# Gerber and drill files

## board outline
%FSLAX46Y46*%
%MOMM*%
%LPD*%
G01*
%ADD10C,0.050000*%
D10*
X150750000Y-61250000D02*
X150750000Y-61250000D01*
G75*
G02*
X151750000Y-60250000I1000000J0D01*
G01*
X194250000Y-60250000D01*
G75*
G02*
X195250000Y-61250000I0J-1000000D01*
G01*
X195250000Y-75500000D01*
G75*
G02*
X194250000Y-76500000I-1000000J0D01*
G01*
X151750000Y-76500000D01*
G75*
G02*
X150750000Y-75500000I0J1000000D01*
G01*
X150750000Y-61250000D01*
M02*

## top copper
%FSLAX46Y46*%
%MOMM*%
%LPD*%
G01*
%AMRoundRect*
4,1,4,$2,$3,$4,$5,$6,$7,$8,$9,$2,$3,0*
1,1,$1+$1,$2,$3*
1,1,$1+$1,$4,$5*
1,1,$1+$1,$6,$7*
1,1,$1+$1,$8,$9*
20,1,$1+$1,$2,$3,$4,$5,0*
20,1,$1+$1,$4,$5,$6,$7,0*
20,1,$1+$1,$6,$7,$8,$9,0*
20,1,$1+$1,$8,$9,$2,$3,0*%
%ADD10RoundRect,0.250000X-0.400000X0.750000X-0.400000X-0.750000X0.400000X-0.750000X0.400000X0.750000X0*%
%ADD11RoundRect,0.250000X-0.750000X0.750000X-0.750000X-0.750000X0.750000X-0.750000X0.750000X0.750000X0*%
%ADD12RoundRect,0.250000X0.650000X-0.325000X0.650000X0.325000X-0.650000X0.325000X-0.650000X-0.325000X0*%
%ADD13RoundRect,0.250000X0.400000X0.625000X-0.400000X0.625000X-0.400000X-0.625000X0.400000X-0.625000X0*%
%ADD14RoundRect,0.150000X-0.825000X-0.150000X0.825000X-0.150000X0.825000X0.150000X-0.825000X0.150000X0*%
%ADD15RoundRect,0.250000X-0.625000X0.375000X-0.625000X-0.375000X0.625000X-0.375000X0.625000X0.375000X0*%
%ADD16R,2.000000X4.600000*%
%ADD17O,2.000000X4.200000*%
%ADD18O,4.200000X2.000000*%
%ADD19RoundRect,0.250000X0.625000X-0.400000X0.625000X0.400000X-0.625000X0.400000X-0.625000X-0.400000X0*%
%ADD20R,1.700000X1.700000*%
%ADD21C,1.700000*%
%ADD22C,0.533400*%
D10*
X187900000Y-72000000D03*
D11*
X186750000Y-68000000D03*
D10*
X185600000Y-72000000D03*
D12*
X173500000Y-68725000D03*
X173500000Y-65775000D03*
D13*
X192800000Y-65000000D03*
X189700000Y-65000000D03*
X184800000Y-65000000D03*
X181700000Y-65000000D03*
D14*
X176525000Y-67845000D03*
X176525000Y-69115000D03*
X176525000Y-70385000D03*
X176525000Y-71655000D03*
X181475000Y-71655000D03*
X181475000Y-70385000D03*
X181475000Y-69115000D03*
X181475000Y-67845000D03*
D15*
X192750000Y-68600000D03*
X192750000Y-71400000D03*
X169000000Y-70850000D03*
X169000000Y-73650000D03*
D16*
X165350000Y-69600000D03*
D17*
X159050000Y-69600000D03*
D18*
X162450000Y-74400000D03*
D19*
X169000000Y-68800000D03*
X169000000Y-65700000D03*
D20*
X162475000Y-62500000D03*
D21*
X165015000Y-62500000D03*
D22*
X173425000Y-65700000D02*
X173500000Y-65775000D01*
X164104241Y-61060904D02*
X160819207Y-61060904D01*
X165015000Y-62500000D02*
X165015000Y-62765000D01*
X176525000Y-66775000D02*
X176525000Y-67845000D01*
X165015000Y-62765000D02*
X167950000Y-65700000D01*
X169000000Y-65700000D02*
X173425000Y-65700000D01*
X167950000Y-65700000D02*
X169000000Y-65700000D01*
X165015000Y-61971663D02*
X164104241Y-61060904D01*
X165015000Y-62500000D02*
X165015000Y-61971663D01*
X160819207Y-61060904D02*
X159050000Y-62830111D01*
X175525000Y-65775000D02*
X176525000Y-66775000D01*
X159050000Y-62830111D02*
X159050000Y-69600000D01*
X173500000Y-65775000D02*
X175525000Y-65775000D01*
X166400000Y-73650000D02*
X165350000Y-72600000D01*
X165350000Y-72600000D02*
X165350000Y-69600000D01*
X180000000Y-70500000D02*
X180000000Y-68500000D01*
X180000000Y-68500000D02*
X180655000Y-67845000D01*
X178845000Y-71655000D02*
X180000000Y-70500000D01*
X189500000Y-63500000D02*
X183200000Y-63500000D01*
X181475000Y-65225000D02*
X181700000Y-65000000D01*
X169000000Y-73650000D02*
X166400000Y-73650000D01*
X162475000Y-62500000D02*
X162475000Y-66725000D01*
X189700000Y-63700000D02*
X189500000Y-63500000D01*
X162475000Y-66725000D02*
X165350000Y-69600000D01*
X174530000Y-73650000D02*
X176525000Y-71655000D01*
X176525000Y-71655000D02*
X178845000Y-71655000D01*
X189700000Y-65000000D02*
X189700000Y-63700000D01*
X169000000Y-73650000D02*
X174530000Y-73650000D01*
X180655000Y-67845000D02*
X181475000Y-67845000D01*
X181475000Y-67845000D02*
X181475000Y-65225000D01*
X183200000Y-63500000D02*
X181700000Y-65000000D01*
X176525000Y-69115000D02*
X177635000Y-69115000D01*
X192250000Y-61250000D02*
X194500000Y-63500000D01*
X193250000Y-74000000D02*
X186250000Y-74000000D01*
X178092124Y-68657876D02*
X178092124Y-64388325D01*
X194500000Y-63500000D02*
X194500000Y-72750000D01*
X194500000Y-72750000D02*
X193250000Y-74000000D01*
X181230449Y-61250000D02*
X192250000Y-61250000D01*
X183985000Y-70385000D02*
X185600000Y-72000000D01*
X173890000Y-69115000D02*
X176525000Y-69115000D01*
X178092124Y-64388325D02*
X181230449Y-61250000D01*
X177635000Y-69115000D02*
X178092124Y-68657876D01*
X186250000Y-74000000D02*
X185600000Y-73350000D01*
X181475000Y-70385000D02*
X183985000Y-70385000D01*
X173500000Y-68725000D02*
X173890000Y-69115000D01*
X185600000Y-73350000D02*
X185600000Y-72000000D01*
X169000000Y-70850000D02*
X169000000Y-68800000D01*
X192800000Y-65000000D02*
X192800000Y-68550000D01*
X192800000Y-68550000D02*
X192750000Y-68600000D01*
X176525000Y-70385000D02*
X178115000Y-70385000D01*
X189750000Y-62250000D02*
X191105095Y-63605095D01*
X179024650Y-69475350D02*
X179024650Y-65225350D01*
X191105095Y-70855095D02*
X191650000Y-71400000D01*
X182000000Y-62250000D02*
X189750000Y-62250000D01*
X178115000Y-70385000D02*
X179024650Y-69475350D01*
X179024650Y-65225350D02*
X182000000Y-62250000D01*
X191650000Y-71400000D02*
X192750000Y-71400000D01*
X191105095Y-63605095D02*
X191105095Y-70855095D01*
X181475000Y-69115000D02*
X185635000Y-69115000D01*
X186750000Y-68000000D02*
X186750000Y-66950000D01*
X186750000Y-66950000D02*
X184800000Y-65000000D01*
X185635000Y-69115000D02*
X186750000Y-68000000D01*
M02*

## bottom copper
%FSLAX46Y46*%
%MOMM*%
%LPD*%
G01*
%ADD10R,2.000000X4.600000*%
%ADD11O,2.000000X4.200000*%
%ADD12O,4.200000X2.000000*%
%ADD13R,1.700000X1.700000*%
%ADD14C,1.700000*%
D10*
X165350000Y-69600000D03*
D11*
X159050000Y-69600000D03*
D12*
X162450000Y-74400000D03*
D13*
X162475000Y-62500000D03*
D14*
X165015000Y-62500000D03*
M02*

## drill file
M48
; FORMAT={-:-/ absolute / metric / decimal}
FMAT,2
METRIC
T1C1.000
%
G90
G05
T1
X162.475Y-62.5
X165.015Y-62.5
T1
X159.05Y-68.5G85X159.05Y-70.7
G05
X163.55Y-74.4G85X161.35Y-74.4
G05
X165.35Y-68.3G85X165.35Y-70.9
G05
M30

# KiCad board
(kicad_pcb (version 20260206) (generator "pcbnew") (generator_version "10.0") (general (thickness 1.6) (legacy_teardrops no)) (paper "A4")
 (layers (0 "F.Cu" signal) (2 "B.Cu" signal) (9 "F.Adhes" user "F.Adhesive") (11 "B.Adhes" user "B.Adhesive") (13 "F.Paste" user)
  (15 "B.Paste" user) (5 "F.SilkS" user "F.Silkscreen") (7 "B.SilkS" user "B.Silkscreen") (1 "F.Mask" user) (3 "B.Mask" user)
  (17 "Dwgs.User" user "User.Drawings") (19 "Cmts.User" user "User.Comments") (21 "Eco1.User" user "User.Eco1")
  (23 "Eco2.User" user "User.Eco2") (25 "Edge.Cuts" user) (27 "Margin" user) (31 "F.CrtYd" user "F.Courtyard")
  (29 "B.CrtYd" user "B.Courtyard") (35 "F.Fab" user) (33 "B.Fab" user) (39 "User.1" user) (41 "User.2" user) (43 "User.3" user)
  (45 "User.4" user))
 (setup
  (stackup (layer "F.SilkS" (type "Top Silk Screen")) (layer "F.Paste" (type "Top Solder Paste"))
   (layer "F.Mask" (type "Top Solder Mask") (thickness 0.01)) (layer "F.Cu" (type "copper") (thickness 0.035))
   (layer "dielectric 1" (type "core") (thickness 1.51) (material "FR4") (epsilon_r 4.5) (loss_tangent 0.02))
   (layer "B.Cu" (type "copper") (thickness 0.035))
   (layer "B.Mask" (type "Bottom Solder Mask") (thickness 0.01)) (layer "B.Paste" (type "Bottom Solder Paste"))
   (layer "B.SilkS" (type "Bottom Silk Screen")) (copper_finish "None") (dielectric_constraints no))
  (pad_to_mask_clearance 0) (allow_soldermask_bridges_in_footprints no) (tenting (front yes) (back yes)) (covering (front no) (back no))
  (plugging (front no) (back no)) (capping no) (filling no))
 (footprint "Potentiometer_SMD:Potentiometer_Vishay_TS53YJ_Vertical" (layer "F.Cu") (at 186.75 70 -90)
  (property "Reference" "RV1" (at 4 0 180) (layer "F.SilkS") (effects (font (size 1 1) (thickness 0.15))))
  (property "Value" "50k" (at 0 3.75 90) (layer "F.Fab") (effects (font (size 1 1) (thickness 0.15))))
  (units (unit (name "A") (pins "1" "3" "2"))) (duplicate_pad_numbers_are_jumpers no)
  (pad "1" smd roundrect (at 2 -1.15 270) (size 2 1.3) (layers "F.Cu" "F.Mask" "F.Paste") (roundrect_rratio 0.192308)
   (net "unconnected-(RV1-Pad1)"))
  (pad "2" smd roundrect (at -2 0 270) (size 2 2) (layers "F.Cu" "F.Mask" "F.Paste") (roundrect_rratio 0.125) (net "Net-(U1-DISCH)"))
  (pad "3" smd roundrect (at 2 1.15 270) (size 2 1.3) (layers "F.Cu" "F.Mask" "F.Paste") (roundrect_rratio 0.192308) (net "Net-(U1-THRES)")))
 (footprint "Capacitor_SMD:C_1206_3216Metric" (layer "F.Cu") (at 173.5 67.25 90)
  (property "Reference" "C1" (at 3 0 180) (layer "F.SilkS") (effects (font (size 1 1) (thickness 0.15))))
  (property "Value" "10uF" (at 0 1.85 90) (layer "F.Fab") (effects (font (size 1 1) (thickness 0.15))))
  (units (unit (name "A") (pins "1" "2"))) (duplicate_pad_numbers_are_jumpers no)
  (pad "1" smd roundrect (at -1.475 0 90) (size 1.15 1.8) (layers "F.Cu" "F.Mask" "F.Paste") (roundrect_rratio 0.217391)
   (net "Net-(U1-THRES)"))
  (pad "2" smd roundrect (at 1.475 0 90) (size 1.15 1.8) (layers "F.Cu" "F.Mask" "F.Paste") (roundrect_rratio 0.217391) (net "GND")))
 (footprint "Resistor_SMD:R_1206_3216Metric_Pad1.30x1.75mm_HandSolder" (layer "F.Cu") (at 191.25 65 180)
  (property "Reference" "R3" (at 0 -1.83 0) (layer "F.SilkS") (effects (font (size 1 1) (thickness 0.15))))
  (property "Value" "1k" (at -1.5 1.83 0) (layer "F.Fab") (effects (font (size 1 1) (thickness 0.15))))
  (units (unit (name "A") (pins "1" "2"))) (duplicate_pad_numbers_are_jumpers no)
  (pad "1" smd roundrect (at -1.55 0 180) (size 1.3 1.75) (layers "F.Cu" "F.Mask" "F.Paste") (roundrect_rratio 0.192308) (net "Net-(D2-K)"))
  (pad "2" smd roundrect (at 1.55 0 180) (size 1.3 1.75) (layers "F.Cu" "F.Mask" "F.Paste") (roundrect_rratio 0.192308) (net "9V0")))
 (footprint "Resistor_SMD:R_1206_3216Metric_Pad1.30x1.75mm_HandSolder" (layer "F.Cu") (at 183.25 65 180)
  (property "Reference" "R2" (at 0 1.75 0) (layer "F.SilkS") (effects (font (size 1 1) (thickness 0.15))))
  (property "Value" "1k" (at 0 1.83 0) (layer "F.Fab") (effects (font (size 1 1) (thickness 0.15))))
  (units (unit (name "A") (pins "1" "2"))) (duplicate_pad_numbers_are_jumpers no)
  (pad "1" smd roundrect (at -1.55 0 180) (size 1.3 1.75) (layers "F.Cu" "F.Mask" "F.Paste") (roundrect_rratio 0.192308)
   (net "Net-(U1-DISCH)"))
  (pad "2" smd roundrect (at 1.55 0 180) (size 1.3 1.75) (layers "F.Cu" "F.Mask" "F.Paste") (roundrect_rratio 0.192308) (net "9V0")))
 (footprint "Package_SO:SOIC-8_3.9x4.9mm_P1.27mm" (layer "F.Cu") (at 179 69.75)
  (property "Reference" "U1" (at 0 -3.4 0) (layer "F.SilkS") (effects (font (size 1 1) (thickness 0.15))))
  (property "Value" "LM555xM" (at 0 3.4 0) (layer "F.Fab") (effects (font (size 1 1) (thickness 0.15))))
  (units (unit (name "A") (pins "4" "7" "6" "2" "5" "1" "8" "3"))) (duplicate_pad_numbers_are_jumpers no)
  (pad "1" smd roundrect (at -2.475 -1.905) (size 1.95 0.6) (layers "F.Cu" "F.Mask" "F.Paste") (roundrect_rratio 0.25) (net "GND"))
  (pad "2" smd roundrect (at -2.475 -0.635) (size 1.95 0.6) (layers "F.Cu" "F.Mask" "F.Paste") (roundrect_rratio 0.25)
   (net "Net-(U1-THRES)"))
  (pad "3" smd roundrect (at -2.475 0.635) (size 1.95 0.6) (layers "F.Cu" "F.Mask" "F.Paste") (roundrect_rratio 0.25) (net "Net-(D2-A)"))
  (pad "4" smd roundrect (at -2.475 1.905) (size 1.95 0.6) (layers "F.Cu" "F.Mask" "F.Paste") (roundrect_rratio 0.25) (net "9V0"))
  (pad "5" smd roundrect (at 2.475 1.905) (size 1.95 0.6) (layers "F.Cu" "F.Mask" "F.Paste") (roundrect_rratio 0.25)
   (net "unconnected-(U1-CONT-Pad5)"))
  (pad "6" smd roundrect (at 2.475 0.635) (size 1.95 0.6) (layers "F.Cu" "F.Mask" "F.Paste") (roundrect_rratio 0.25) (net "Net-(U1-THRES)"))
  (pad "7" smd roundrect (at 2.475 -0.635) (size 1.95 0.6) (layers "F.Cu" "F.Mask" "F.Paste") (roundrect_rratio 0.25) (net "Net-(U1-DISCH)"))
  (pad "8" smd roundrect (at 2.475 -1.905) (size 1.95 0.6) (layers "F.Cu" "F.Mask" "F.Paste") (roundrect_rratio 0.25) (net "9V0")))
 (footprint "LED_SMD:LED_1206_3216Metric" (layer "F.Cu") (at 192.75 70 -90)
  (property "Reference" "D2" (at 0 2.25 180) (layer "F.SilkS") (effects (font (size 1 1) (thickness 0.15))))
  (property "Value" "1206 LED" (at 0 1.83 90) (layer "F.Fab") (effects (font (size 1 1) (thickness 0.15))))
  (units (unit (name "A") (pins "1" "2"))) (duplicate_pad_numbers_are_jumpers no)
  (pad "1" smd roundrect (at -1.4 0 270) (size 1.25 1.75) (layers "F.Cu" "F.Mask" "F.Paste") (roundrect_rratio 0.2) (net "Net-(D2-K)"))
  (pad "2" smd roundrect (at 1.4 0 270) (size 1.25 1.75) (layers "F.Cu" "F.Mask" "F.Paste") (roundrect_rratio 0.2) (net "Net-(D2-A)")))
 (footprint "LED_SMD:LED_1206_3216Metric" (layer "F.Cu") (at 169 72.25 -90)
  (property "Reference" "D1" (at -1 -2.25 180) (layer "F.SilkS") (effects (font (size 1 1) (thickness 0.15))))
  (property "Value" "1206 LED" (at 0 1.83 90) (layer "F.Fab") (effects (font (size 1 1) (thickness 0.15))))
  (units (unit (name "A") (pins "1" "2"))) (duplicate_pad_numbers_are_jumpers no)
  (pad "1" smd roundrect (at -1.4 0 270) (size 1.25 1.75) (layers "F.Cu" "F.Mask" "F.Paste") (roundrect_rratio 0.2) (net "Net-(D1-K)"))
  (pad "2" smd roundrect (at 1.4 0 270) (size 1.25 1.75) (layers "F.Cu" "F.Mask" "F.Paste") (roundrect_rratio 0.2) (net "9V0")))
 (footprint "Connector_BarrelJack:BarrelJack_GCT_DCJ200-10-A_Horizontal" (layer "F.Cu") (at 165.35 69.6 -90)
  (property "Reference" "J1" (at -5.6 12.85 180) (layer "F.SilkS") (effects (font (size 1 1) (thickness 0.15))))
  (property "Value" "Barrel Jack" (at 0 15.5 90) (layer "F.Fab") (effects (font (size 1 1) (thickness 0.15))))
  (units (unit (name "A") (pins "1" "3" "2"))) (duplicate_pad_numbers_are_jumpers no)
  (pad "1" thru_hole rect (at 0 0 270) (size 4.6 2) (drill oval 3.6 1) (layers "*.Cu" "*.Mask") (remove_unused_layers no) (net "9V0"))
  (pad "2" thru_hole oval (at 0 6.3 270) (size 4.2 2) (drill oval 3.2 1) (layers "*.Cu" "*.Mask") (remove_unused_layers no) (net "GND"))
  (pad "3" thru_hole oval (at 4.8 2.9 270) (size 2 4.2) (drill oval 1 3.2) (layers "*.Cu" "*.Mask") (remove_unused_layers no)
   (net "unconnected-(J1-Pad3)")))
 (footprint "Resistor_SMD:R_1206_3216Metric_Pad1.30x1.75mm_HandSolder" (layer "F.Cu") (at 169 67.25 90)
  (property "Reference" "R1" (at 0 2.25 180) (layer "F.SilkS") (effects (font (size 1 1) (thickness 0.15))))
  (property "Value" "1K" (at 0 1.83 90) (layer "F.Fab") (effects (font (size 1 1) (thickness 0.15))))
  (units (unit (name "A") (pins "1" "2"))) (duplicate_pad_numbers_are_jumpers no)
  (pad "1" smd roundrect (at -1.55 0 90) (size 1.3 1.75) (layers "F.Cu" "F.Mask" "F.Paste") (roundrect_rratio 0.192308) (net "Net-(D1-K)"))
  (pad "2" smd roundrect (at 1.55 0 90) (size 1.3 1.75) (layers "F.Cu" "F.Mask" "F.Paste") (roundrect_rratio 0.192308) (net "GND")))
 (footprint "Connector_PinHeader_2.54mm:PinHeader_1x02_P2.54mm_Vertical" (layer "F.Cu") (at 162.475 62.5 90)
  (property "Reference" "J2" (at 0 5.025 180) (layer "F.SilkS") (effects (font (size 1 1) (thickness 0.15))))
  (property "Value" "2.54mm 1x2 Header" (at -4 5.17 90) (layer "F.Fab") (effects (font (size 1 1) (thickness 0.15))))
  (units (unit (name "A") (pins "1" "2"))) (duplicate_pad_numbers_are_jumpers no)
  (pad "1" thru_hole rect (at 0 0 90) (size 1.7 1.7) (drill 1) (layers "*.Cu" "*.Mask") (remove_unused_layers no) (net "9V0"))
  (pad "2" thru_hole circle (at 0 2.54 90) (size 1.7 1.7) (drill 1) (layers "*.Cu" "*.Mask") (remove_unused_layers no) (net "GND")))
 (gr_rect (start 150.75 60.25) (end 195.25 76.5) (radius 1) (stroke (width 0.05) (type solid)) (fill no) (layer "Edge.Cuts"))
 (segment (start 173.425 65.7) (end 173.5 65.775) (width 0.5334) (layer "F.Cu") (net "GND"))
 (segment (start 164.104241 61.060904) (end 160.819207 61.060904) (width 0.5334) (layer "F.Cu") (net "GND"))
 (segment (start 165.015 62.5) (end 165.015 62.765) (width 0.5334) (layer "F.Cu") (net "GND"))
 (segment (start 176.525 66.775) (end 176.525 67.845) (width 0.5334) (layer "F.Cu") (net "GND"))
 (segment (start 165.015 62.765) (end 167.95 65.7) (width 0.5334) (layer "F.Cu") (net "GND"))
 (segment (start 169 65.7) (end 173.425 65.7) (width 0.5334) (layer "F.Cu") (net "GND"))
 (segment (start 167.95 65.7) (end 169 65.7) (width 0.5334) (layer "F.Cu") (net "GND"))
 (segment (start 165.015 61.971663) (end 164.104241 61.060904) (width 0.5334) (layer "F.Cu") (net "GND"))
 (segment (start 165.015 62.5) (end 165.015 61.971663) (width 0.5334) (layer "F.Cu") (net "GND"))
 (segment (start 160.819207 61.060904) (end 159.05 62.830111) (width 0.5334) (layer "F.Cu") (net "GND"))
 (segment (start 175.525 65.775) (end 176.525 66.775) (width 0.5334) (layer "F.Cu") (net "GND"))
 (segment (start 159.05 62.830111) (end 159.05 69.6) (width 0.5334) (layer "F.Cu") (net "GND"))
 (segment (start 173.5 65.775) (end 175.525 65.775) (width 0.5334) (layer "F.Cu") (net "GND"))
 (segment (start 166.4 73.65) (end 165.35 72.6) (width 0.5334) (layer "F.Cu") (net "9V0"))
 (segment (start 165.35 72.6) (end 165.35 69.6) (width 0.5334) (layer "F.Cu") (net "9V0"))
 (segment (start 180 70.5) (end 180 68.5) (width 0.5334) (layer "F.Cu") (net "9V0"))
 (segment (start 180 68.5) (end 180.655 67.845) (width 0.5334) (layer "F.Cu") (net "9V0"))
 (segment (start 178.845 71.655) (end 180 70.5) (width 0.5334) (layer "F.Cu") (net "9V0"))
 (segment (start 189.5 63.5) (end 183.2 63.5) (width 0.5334) (layer "F.Cu") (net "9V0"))
 (segment (start 181.475 65.225) (end 181.7 65) (width 0.5334) (layer "F.Cu") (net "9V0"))
 (segment (start 169 73.65) (end 166.4 73.65) (width 0.5334) (layer "F.Cu") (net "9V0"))
 (segment (start 162.475 62.5) (end 162.475 66.725) (width 0.5334) (layer "F.Cu") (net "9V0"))
 (segment (start 189.7 63.7) (end 189.5 63.5) (width 0.5334) (layer "F.Cu") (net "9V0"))
 (segment (start 162.475 66.725) (end 165.35 69.6) (width 0.5334) (layer "F.Cu") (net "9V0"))
 (segment (start 174.53 73.65) (end 176.525 71.655) (width 0.5334) (layer "F.Cu") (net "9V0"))
 (segment (start 176.525 71.655) (end 178.845 71.655) (width 0.5334) (layer "F.Cu") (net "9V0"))
 (segment (start 189.7 65) (end 189.7 63.7) (width 0.5334) (layer "F.Cu") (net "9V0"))
 (segment (start 169 73.65) (end 174.53 73.65) (width 0.5334) (layer "F.Cu") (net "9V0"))
 (segment (start 180.655 67.845) (end 181.475 67.845) (width 0.5334) (layer "F.Cu") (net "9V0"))
 (segment (start 181.475 67.845) (end 181.475 65.225) (width 0.5334) (layer "F.Cu") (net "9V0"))
 (segment (start 183.2 63.5) (end 181.7 65) (width 0.5334) (layer "F.Cu") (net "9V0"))
 (segment (start 176.525 69.115) (end 177.635 69.115) (width 0.5334) (layer "F.Cu") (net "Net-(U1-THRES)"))
 (segment (start 192.25 61.25) (end 194.5 63.5) (width 0.5334) (layer "F.Cu") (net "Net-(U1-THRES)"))
 (segment (start 193.25 74) (end 186.25 74) (width 0.5334) (layer "F.Cu") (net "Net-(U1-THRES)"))
 (segment (start 178.092124 68.657876) (end 178.092124 64.388325) (width 0.5334) (layer "F.Cu") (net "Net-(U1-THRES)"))
 (segment (start 194.5 63.5) (end 194.5 72.75) (width 0.5334) (layer "F.Cu") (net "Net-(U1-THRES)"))
 (segment (start 194.5 72.75) (end 193.25 74) (width 0.5334) (layer "F.Cu") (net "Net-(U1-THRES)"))
 (segment (start 181.230449 61.25) (end 192.25 61.25) (width 0.5334) (layer "F.Cu") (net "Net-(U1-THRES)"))
 (segment (start 183.985 70.385) (end 185.6 72) (width 0.5334) (layer "F.Cu") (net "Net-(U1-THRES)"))
 (segment (start 173.89 69.115) (end 176.525 69.115) (width 0.5334) (layer "F.Cu") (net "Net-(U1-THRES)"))
 (segment (start 178.092124 64.388325) (end 181.230449 61.25) (width 0.5334) (layer "F.Cu") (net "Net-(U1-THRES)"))
 (segment (start 177.635 69.115) (end 178.092124 68.657876) (width 0.5334) (layer "F.Cu") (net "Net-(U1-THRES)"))
 (segment (start 186.25 74) (end 185.6 73.35) (width 0.5334) (layer "F.Cu") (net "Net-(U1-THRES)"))
 (segment (start 181.475 70.385) (end 183.985 70.385) (width 0.5334) (layer "F.Cu") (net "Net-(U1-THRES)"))
 (segment (start 173.5 68.725) (end 173.89 69.115) (width 0.5334) (layer "F.Cu") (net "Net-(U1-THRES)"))
 (segment (start 185.6 73.35) (end 185.6 72) (width 0.5334) (layer "F.Cu") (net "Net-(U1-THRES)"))
 (segment (start 169 70.85) (end 169 68.8) (width 0.5334) (layer "F.Cu") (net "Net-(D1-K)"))
 (segment (start 192.8 65) (end 192.8 68.55) (width 0.5334) (layer "F.Cu") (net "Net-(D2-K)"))
 (segment (start 192.8 68.55) (end 192.75 68.6) (width 0.5334) (layer "F.Cu") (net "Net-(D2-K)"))
 (segment (start 176.525 70.385) (end 178.115 70.385) (width 0.5334) (layer "F.Cu") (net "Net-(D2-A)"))
 (segment (start 189.75 62.25) (end 191.105095 63.605095) (width 0.5334) (layer "F.Cu") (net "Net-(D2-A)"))
 (segment (start 179.02465 69.47535) (end 179.02465 65.22535) (width 0.5334) (layer "F.Cu") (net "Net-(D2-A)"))
 (segment (start 191.105095 70.855095) (end 191.65 71.4) (width 0.5334) (layer "F.Cu") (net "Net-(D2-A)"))
 (segment (start 182 62.25) (end 189.75 62.25) (width 0.5334) (layer "F.Cu") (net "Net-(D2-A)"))
 (segment (start 178.115 70.385) (end 179.02465 69.47535) (width 0.5334) (layer "F.Cu") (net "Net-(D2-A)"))
 (segment (start 179.02465 65.22535) (end 182 62.25) (width 0.5334) (layer "F.Cu") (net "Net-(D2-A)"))
 (segment (start 191.65 71.4) (end 192.75 71.4) (width 0.5334) (layer "F.Cu") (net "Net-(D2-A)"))
 (segment (start 191.105095 63.605095) (end 191.105095 70.855095) (width 0.5334) (layer "F.Cu") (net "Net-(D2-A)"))
 (segment (start 181.475 69.115) (end 185.635 69.115) (width 0.5334) (layer "F.Cu") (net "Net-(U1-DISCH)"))
 (segment (start 186.75 68) (end 186.75 66.95) (width 0.5334) (layer "F.Cu") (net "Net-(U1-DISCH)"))
 (segment (start 186.75 66.95) (end 184.8 65) (width 0.5334) (layer "F.Cu") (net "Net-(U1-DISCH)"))
 (segment (start 185.635 69.115) (end 186.75 68) (width 0.5334) (layer "F.Cu") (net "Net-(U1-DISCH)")))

